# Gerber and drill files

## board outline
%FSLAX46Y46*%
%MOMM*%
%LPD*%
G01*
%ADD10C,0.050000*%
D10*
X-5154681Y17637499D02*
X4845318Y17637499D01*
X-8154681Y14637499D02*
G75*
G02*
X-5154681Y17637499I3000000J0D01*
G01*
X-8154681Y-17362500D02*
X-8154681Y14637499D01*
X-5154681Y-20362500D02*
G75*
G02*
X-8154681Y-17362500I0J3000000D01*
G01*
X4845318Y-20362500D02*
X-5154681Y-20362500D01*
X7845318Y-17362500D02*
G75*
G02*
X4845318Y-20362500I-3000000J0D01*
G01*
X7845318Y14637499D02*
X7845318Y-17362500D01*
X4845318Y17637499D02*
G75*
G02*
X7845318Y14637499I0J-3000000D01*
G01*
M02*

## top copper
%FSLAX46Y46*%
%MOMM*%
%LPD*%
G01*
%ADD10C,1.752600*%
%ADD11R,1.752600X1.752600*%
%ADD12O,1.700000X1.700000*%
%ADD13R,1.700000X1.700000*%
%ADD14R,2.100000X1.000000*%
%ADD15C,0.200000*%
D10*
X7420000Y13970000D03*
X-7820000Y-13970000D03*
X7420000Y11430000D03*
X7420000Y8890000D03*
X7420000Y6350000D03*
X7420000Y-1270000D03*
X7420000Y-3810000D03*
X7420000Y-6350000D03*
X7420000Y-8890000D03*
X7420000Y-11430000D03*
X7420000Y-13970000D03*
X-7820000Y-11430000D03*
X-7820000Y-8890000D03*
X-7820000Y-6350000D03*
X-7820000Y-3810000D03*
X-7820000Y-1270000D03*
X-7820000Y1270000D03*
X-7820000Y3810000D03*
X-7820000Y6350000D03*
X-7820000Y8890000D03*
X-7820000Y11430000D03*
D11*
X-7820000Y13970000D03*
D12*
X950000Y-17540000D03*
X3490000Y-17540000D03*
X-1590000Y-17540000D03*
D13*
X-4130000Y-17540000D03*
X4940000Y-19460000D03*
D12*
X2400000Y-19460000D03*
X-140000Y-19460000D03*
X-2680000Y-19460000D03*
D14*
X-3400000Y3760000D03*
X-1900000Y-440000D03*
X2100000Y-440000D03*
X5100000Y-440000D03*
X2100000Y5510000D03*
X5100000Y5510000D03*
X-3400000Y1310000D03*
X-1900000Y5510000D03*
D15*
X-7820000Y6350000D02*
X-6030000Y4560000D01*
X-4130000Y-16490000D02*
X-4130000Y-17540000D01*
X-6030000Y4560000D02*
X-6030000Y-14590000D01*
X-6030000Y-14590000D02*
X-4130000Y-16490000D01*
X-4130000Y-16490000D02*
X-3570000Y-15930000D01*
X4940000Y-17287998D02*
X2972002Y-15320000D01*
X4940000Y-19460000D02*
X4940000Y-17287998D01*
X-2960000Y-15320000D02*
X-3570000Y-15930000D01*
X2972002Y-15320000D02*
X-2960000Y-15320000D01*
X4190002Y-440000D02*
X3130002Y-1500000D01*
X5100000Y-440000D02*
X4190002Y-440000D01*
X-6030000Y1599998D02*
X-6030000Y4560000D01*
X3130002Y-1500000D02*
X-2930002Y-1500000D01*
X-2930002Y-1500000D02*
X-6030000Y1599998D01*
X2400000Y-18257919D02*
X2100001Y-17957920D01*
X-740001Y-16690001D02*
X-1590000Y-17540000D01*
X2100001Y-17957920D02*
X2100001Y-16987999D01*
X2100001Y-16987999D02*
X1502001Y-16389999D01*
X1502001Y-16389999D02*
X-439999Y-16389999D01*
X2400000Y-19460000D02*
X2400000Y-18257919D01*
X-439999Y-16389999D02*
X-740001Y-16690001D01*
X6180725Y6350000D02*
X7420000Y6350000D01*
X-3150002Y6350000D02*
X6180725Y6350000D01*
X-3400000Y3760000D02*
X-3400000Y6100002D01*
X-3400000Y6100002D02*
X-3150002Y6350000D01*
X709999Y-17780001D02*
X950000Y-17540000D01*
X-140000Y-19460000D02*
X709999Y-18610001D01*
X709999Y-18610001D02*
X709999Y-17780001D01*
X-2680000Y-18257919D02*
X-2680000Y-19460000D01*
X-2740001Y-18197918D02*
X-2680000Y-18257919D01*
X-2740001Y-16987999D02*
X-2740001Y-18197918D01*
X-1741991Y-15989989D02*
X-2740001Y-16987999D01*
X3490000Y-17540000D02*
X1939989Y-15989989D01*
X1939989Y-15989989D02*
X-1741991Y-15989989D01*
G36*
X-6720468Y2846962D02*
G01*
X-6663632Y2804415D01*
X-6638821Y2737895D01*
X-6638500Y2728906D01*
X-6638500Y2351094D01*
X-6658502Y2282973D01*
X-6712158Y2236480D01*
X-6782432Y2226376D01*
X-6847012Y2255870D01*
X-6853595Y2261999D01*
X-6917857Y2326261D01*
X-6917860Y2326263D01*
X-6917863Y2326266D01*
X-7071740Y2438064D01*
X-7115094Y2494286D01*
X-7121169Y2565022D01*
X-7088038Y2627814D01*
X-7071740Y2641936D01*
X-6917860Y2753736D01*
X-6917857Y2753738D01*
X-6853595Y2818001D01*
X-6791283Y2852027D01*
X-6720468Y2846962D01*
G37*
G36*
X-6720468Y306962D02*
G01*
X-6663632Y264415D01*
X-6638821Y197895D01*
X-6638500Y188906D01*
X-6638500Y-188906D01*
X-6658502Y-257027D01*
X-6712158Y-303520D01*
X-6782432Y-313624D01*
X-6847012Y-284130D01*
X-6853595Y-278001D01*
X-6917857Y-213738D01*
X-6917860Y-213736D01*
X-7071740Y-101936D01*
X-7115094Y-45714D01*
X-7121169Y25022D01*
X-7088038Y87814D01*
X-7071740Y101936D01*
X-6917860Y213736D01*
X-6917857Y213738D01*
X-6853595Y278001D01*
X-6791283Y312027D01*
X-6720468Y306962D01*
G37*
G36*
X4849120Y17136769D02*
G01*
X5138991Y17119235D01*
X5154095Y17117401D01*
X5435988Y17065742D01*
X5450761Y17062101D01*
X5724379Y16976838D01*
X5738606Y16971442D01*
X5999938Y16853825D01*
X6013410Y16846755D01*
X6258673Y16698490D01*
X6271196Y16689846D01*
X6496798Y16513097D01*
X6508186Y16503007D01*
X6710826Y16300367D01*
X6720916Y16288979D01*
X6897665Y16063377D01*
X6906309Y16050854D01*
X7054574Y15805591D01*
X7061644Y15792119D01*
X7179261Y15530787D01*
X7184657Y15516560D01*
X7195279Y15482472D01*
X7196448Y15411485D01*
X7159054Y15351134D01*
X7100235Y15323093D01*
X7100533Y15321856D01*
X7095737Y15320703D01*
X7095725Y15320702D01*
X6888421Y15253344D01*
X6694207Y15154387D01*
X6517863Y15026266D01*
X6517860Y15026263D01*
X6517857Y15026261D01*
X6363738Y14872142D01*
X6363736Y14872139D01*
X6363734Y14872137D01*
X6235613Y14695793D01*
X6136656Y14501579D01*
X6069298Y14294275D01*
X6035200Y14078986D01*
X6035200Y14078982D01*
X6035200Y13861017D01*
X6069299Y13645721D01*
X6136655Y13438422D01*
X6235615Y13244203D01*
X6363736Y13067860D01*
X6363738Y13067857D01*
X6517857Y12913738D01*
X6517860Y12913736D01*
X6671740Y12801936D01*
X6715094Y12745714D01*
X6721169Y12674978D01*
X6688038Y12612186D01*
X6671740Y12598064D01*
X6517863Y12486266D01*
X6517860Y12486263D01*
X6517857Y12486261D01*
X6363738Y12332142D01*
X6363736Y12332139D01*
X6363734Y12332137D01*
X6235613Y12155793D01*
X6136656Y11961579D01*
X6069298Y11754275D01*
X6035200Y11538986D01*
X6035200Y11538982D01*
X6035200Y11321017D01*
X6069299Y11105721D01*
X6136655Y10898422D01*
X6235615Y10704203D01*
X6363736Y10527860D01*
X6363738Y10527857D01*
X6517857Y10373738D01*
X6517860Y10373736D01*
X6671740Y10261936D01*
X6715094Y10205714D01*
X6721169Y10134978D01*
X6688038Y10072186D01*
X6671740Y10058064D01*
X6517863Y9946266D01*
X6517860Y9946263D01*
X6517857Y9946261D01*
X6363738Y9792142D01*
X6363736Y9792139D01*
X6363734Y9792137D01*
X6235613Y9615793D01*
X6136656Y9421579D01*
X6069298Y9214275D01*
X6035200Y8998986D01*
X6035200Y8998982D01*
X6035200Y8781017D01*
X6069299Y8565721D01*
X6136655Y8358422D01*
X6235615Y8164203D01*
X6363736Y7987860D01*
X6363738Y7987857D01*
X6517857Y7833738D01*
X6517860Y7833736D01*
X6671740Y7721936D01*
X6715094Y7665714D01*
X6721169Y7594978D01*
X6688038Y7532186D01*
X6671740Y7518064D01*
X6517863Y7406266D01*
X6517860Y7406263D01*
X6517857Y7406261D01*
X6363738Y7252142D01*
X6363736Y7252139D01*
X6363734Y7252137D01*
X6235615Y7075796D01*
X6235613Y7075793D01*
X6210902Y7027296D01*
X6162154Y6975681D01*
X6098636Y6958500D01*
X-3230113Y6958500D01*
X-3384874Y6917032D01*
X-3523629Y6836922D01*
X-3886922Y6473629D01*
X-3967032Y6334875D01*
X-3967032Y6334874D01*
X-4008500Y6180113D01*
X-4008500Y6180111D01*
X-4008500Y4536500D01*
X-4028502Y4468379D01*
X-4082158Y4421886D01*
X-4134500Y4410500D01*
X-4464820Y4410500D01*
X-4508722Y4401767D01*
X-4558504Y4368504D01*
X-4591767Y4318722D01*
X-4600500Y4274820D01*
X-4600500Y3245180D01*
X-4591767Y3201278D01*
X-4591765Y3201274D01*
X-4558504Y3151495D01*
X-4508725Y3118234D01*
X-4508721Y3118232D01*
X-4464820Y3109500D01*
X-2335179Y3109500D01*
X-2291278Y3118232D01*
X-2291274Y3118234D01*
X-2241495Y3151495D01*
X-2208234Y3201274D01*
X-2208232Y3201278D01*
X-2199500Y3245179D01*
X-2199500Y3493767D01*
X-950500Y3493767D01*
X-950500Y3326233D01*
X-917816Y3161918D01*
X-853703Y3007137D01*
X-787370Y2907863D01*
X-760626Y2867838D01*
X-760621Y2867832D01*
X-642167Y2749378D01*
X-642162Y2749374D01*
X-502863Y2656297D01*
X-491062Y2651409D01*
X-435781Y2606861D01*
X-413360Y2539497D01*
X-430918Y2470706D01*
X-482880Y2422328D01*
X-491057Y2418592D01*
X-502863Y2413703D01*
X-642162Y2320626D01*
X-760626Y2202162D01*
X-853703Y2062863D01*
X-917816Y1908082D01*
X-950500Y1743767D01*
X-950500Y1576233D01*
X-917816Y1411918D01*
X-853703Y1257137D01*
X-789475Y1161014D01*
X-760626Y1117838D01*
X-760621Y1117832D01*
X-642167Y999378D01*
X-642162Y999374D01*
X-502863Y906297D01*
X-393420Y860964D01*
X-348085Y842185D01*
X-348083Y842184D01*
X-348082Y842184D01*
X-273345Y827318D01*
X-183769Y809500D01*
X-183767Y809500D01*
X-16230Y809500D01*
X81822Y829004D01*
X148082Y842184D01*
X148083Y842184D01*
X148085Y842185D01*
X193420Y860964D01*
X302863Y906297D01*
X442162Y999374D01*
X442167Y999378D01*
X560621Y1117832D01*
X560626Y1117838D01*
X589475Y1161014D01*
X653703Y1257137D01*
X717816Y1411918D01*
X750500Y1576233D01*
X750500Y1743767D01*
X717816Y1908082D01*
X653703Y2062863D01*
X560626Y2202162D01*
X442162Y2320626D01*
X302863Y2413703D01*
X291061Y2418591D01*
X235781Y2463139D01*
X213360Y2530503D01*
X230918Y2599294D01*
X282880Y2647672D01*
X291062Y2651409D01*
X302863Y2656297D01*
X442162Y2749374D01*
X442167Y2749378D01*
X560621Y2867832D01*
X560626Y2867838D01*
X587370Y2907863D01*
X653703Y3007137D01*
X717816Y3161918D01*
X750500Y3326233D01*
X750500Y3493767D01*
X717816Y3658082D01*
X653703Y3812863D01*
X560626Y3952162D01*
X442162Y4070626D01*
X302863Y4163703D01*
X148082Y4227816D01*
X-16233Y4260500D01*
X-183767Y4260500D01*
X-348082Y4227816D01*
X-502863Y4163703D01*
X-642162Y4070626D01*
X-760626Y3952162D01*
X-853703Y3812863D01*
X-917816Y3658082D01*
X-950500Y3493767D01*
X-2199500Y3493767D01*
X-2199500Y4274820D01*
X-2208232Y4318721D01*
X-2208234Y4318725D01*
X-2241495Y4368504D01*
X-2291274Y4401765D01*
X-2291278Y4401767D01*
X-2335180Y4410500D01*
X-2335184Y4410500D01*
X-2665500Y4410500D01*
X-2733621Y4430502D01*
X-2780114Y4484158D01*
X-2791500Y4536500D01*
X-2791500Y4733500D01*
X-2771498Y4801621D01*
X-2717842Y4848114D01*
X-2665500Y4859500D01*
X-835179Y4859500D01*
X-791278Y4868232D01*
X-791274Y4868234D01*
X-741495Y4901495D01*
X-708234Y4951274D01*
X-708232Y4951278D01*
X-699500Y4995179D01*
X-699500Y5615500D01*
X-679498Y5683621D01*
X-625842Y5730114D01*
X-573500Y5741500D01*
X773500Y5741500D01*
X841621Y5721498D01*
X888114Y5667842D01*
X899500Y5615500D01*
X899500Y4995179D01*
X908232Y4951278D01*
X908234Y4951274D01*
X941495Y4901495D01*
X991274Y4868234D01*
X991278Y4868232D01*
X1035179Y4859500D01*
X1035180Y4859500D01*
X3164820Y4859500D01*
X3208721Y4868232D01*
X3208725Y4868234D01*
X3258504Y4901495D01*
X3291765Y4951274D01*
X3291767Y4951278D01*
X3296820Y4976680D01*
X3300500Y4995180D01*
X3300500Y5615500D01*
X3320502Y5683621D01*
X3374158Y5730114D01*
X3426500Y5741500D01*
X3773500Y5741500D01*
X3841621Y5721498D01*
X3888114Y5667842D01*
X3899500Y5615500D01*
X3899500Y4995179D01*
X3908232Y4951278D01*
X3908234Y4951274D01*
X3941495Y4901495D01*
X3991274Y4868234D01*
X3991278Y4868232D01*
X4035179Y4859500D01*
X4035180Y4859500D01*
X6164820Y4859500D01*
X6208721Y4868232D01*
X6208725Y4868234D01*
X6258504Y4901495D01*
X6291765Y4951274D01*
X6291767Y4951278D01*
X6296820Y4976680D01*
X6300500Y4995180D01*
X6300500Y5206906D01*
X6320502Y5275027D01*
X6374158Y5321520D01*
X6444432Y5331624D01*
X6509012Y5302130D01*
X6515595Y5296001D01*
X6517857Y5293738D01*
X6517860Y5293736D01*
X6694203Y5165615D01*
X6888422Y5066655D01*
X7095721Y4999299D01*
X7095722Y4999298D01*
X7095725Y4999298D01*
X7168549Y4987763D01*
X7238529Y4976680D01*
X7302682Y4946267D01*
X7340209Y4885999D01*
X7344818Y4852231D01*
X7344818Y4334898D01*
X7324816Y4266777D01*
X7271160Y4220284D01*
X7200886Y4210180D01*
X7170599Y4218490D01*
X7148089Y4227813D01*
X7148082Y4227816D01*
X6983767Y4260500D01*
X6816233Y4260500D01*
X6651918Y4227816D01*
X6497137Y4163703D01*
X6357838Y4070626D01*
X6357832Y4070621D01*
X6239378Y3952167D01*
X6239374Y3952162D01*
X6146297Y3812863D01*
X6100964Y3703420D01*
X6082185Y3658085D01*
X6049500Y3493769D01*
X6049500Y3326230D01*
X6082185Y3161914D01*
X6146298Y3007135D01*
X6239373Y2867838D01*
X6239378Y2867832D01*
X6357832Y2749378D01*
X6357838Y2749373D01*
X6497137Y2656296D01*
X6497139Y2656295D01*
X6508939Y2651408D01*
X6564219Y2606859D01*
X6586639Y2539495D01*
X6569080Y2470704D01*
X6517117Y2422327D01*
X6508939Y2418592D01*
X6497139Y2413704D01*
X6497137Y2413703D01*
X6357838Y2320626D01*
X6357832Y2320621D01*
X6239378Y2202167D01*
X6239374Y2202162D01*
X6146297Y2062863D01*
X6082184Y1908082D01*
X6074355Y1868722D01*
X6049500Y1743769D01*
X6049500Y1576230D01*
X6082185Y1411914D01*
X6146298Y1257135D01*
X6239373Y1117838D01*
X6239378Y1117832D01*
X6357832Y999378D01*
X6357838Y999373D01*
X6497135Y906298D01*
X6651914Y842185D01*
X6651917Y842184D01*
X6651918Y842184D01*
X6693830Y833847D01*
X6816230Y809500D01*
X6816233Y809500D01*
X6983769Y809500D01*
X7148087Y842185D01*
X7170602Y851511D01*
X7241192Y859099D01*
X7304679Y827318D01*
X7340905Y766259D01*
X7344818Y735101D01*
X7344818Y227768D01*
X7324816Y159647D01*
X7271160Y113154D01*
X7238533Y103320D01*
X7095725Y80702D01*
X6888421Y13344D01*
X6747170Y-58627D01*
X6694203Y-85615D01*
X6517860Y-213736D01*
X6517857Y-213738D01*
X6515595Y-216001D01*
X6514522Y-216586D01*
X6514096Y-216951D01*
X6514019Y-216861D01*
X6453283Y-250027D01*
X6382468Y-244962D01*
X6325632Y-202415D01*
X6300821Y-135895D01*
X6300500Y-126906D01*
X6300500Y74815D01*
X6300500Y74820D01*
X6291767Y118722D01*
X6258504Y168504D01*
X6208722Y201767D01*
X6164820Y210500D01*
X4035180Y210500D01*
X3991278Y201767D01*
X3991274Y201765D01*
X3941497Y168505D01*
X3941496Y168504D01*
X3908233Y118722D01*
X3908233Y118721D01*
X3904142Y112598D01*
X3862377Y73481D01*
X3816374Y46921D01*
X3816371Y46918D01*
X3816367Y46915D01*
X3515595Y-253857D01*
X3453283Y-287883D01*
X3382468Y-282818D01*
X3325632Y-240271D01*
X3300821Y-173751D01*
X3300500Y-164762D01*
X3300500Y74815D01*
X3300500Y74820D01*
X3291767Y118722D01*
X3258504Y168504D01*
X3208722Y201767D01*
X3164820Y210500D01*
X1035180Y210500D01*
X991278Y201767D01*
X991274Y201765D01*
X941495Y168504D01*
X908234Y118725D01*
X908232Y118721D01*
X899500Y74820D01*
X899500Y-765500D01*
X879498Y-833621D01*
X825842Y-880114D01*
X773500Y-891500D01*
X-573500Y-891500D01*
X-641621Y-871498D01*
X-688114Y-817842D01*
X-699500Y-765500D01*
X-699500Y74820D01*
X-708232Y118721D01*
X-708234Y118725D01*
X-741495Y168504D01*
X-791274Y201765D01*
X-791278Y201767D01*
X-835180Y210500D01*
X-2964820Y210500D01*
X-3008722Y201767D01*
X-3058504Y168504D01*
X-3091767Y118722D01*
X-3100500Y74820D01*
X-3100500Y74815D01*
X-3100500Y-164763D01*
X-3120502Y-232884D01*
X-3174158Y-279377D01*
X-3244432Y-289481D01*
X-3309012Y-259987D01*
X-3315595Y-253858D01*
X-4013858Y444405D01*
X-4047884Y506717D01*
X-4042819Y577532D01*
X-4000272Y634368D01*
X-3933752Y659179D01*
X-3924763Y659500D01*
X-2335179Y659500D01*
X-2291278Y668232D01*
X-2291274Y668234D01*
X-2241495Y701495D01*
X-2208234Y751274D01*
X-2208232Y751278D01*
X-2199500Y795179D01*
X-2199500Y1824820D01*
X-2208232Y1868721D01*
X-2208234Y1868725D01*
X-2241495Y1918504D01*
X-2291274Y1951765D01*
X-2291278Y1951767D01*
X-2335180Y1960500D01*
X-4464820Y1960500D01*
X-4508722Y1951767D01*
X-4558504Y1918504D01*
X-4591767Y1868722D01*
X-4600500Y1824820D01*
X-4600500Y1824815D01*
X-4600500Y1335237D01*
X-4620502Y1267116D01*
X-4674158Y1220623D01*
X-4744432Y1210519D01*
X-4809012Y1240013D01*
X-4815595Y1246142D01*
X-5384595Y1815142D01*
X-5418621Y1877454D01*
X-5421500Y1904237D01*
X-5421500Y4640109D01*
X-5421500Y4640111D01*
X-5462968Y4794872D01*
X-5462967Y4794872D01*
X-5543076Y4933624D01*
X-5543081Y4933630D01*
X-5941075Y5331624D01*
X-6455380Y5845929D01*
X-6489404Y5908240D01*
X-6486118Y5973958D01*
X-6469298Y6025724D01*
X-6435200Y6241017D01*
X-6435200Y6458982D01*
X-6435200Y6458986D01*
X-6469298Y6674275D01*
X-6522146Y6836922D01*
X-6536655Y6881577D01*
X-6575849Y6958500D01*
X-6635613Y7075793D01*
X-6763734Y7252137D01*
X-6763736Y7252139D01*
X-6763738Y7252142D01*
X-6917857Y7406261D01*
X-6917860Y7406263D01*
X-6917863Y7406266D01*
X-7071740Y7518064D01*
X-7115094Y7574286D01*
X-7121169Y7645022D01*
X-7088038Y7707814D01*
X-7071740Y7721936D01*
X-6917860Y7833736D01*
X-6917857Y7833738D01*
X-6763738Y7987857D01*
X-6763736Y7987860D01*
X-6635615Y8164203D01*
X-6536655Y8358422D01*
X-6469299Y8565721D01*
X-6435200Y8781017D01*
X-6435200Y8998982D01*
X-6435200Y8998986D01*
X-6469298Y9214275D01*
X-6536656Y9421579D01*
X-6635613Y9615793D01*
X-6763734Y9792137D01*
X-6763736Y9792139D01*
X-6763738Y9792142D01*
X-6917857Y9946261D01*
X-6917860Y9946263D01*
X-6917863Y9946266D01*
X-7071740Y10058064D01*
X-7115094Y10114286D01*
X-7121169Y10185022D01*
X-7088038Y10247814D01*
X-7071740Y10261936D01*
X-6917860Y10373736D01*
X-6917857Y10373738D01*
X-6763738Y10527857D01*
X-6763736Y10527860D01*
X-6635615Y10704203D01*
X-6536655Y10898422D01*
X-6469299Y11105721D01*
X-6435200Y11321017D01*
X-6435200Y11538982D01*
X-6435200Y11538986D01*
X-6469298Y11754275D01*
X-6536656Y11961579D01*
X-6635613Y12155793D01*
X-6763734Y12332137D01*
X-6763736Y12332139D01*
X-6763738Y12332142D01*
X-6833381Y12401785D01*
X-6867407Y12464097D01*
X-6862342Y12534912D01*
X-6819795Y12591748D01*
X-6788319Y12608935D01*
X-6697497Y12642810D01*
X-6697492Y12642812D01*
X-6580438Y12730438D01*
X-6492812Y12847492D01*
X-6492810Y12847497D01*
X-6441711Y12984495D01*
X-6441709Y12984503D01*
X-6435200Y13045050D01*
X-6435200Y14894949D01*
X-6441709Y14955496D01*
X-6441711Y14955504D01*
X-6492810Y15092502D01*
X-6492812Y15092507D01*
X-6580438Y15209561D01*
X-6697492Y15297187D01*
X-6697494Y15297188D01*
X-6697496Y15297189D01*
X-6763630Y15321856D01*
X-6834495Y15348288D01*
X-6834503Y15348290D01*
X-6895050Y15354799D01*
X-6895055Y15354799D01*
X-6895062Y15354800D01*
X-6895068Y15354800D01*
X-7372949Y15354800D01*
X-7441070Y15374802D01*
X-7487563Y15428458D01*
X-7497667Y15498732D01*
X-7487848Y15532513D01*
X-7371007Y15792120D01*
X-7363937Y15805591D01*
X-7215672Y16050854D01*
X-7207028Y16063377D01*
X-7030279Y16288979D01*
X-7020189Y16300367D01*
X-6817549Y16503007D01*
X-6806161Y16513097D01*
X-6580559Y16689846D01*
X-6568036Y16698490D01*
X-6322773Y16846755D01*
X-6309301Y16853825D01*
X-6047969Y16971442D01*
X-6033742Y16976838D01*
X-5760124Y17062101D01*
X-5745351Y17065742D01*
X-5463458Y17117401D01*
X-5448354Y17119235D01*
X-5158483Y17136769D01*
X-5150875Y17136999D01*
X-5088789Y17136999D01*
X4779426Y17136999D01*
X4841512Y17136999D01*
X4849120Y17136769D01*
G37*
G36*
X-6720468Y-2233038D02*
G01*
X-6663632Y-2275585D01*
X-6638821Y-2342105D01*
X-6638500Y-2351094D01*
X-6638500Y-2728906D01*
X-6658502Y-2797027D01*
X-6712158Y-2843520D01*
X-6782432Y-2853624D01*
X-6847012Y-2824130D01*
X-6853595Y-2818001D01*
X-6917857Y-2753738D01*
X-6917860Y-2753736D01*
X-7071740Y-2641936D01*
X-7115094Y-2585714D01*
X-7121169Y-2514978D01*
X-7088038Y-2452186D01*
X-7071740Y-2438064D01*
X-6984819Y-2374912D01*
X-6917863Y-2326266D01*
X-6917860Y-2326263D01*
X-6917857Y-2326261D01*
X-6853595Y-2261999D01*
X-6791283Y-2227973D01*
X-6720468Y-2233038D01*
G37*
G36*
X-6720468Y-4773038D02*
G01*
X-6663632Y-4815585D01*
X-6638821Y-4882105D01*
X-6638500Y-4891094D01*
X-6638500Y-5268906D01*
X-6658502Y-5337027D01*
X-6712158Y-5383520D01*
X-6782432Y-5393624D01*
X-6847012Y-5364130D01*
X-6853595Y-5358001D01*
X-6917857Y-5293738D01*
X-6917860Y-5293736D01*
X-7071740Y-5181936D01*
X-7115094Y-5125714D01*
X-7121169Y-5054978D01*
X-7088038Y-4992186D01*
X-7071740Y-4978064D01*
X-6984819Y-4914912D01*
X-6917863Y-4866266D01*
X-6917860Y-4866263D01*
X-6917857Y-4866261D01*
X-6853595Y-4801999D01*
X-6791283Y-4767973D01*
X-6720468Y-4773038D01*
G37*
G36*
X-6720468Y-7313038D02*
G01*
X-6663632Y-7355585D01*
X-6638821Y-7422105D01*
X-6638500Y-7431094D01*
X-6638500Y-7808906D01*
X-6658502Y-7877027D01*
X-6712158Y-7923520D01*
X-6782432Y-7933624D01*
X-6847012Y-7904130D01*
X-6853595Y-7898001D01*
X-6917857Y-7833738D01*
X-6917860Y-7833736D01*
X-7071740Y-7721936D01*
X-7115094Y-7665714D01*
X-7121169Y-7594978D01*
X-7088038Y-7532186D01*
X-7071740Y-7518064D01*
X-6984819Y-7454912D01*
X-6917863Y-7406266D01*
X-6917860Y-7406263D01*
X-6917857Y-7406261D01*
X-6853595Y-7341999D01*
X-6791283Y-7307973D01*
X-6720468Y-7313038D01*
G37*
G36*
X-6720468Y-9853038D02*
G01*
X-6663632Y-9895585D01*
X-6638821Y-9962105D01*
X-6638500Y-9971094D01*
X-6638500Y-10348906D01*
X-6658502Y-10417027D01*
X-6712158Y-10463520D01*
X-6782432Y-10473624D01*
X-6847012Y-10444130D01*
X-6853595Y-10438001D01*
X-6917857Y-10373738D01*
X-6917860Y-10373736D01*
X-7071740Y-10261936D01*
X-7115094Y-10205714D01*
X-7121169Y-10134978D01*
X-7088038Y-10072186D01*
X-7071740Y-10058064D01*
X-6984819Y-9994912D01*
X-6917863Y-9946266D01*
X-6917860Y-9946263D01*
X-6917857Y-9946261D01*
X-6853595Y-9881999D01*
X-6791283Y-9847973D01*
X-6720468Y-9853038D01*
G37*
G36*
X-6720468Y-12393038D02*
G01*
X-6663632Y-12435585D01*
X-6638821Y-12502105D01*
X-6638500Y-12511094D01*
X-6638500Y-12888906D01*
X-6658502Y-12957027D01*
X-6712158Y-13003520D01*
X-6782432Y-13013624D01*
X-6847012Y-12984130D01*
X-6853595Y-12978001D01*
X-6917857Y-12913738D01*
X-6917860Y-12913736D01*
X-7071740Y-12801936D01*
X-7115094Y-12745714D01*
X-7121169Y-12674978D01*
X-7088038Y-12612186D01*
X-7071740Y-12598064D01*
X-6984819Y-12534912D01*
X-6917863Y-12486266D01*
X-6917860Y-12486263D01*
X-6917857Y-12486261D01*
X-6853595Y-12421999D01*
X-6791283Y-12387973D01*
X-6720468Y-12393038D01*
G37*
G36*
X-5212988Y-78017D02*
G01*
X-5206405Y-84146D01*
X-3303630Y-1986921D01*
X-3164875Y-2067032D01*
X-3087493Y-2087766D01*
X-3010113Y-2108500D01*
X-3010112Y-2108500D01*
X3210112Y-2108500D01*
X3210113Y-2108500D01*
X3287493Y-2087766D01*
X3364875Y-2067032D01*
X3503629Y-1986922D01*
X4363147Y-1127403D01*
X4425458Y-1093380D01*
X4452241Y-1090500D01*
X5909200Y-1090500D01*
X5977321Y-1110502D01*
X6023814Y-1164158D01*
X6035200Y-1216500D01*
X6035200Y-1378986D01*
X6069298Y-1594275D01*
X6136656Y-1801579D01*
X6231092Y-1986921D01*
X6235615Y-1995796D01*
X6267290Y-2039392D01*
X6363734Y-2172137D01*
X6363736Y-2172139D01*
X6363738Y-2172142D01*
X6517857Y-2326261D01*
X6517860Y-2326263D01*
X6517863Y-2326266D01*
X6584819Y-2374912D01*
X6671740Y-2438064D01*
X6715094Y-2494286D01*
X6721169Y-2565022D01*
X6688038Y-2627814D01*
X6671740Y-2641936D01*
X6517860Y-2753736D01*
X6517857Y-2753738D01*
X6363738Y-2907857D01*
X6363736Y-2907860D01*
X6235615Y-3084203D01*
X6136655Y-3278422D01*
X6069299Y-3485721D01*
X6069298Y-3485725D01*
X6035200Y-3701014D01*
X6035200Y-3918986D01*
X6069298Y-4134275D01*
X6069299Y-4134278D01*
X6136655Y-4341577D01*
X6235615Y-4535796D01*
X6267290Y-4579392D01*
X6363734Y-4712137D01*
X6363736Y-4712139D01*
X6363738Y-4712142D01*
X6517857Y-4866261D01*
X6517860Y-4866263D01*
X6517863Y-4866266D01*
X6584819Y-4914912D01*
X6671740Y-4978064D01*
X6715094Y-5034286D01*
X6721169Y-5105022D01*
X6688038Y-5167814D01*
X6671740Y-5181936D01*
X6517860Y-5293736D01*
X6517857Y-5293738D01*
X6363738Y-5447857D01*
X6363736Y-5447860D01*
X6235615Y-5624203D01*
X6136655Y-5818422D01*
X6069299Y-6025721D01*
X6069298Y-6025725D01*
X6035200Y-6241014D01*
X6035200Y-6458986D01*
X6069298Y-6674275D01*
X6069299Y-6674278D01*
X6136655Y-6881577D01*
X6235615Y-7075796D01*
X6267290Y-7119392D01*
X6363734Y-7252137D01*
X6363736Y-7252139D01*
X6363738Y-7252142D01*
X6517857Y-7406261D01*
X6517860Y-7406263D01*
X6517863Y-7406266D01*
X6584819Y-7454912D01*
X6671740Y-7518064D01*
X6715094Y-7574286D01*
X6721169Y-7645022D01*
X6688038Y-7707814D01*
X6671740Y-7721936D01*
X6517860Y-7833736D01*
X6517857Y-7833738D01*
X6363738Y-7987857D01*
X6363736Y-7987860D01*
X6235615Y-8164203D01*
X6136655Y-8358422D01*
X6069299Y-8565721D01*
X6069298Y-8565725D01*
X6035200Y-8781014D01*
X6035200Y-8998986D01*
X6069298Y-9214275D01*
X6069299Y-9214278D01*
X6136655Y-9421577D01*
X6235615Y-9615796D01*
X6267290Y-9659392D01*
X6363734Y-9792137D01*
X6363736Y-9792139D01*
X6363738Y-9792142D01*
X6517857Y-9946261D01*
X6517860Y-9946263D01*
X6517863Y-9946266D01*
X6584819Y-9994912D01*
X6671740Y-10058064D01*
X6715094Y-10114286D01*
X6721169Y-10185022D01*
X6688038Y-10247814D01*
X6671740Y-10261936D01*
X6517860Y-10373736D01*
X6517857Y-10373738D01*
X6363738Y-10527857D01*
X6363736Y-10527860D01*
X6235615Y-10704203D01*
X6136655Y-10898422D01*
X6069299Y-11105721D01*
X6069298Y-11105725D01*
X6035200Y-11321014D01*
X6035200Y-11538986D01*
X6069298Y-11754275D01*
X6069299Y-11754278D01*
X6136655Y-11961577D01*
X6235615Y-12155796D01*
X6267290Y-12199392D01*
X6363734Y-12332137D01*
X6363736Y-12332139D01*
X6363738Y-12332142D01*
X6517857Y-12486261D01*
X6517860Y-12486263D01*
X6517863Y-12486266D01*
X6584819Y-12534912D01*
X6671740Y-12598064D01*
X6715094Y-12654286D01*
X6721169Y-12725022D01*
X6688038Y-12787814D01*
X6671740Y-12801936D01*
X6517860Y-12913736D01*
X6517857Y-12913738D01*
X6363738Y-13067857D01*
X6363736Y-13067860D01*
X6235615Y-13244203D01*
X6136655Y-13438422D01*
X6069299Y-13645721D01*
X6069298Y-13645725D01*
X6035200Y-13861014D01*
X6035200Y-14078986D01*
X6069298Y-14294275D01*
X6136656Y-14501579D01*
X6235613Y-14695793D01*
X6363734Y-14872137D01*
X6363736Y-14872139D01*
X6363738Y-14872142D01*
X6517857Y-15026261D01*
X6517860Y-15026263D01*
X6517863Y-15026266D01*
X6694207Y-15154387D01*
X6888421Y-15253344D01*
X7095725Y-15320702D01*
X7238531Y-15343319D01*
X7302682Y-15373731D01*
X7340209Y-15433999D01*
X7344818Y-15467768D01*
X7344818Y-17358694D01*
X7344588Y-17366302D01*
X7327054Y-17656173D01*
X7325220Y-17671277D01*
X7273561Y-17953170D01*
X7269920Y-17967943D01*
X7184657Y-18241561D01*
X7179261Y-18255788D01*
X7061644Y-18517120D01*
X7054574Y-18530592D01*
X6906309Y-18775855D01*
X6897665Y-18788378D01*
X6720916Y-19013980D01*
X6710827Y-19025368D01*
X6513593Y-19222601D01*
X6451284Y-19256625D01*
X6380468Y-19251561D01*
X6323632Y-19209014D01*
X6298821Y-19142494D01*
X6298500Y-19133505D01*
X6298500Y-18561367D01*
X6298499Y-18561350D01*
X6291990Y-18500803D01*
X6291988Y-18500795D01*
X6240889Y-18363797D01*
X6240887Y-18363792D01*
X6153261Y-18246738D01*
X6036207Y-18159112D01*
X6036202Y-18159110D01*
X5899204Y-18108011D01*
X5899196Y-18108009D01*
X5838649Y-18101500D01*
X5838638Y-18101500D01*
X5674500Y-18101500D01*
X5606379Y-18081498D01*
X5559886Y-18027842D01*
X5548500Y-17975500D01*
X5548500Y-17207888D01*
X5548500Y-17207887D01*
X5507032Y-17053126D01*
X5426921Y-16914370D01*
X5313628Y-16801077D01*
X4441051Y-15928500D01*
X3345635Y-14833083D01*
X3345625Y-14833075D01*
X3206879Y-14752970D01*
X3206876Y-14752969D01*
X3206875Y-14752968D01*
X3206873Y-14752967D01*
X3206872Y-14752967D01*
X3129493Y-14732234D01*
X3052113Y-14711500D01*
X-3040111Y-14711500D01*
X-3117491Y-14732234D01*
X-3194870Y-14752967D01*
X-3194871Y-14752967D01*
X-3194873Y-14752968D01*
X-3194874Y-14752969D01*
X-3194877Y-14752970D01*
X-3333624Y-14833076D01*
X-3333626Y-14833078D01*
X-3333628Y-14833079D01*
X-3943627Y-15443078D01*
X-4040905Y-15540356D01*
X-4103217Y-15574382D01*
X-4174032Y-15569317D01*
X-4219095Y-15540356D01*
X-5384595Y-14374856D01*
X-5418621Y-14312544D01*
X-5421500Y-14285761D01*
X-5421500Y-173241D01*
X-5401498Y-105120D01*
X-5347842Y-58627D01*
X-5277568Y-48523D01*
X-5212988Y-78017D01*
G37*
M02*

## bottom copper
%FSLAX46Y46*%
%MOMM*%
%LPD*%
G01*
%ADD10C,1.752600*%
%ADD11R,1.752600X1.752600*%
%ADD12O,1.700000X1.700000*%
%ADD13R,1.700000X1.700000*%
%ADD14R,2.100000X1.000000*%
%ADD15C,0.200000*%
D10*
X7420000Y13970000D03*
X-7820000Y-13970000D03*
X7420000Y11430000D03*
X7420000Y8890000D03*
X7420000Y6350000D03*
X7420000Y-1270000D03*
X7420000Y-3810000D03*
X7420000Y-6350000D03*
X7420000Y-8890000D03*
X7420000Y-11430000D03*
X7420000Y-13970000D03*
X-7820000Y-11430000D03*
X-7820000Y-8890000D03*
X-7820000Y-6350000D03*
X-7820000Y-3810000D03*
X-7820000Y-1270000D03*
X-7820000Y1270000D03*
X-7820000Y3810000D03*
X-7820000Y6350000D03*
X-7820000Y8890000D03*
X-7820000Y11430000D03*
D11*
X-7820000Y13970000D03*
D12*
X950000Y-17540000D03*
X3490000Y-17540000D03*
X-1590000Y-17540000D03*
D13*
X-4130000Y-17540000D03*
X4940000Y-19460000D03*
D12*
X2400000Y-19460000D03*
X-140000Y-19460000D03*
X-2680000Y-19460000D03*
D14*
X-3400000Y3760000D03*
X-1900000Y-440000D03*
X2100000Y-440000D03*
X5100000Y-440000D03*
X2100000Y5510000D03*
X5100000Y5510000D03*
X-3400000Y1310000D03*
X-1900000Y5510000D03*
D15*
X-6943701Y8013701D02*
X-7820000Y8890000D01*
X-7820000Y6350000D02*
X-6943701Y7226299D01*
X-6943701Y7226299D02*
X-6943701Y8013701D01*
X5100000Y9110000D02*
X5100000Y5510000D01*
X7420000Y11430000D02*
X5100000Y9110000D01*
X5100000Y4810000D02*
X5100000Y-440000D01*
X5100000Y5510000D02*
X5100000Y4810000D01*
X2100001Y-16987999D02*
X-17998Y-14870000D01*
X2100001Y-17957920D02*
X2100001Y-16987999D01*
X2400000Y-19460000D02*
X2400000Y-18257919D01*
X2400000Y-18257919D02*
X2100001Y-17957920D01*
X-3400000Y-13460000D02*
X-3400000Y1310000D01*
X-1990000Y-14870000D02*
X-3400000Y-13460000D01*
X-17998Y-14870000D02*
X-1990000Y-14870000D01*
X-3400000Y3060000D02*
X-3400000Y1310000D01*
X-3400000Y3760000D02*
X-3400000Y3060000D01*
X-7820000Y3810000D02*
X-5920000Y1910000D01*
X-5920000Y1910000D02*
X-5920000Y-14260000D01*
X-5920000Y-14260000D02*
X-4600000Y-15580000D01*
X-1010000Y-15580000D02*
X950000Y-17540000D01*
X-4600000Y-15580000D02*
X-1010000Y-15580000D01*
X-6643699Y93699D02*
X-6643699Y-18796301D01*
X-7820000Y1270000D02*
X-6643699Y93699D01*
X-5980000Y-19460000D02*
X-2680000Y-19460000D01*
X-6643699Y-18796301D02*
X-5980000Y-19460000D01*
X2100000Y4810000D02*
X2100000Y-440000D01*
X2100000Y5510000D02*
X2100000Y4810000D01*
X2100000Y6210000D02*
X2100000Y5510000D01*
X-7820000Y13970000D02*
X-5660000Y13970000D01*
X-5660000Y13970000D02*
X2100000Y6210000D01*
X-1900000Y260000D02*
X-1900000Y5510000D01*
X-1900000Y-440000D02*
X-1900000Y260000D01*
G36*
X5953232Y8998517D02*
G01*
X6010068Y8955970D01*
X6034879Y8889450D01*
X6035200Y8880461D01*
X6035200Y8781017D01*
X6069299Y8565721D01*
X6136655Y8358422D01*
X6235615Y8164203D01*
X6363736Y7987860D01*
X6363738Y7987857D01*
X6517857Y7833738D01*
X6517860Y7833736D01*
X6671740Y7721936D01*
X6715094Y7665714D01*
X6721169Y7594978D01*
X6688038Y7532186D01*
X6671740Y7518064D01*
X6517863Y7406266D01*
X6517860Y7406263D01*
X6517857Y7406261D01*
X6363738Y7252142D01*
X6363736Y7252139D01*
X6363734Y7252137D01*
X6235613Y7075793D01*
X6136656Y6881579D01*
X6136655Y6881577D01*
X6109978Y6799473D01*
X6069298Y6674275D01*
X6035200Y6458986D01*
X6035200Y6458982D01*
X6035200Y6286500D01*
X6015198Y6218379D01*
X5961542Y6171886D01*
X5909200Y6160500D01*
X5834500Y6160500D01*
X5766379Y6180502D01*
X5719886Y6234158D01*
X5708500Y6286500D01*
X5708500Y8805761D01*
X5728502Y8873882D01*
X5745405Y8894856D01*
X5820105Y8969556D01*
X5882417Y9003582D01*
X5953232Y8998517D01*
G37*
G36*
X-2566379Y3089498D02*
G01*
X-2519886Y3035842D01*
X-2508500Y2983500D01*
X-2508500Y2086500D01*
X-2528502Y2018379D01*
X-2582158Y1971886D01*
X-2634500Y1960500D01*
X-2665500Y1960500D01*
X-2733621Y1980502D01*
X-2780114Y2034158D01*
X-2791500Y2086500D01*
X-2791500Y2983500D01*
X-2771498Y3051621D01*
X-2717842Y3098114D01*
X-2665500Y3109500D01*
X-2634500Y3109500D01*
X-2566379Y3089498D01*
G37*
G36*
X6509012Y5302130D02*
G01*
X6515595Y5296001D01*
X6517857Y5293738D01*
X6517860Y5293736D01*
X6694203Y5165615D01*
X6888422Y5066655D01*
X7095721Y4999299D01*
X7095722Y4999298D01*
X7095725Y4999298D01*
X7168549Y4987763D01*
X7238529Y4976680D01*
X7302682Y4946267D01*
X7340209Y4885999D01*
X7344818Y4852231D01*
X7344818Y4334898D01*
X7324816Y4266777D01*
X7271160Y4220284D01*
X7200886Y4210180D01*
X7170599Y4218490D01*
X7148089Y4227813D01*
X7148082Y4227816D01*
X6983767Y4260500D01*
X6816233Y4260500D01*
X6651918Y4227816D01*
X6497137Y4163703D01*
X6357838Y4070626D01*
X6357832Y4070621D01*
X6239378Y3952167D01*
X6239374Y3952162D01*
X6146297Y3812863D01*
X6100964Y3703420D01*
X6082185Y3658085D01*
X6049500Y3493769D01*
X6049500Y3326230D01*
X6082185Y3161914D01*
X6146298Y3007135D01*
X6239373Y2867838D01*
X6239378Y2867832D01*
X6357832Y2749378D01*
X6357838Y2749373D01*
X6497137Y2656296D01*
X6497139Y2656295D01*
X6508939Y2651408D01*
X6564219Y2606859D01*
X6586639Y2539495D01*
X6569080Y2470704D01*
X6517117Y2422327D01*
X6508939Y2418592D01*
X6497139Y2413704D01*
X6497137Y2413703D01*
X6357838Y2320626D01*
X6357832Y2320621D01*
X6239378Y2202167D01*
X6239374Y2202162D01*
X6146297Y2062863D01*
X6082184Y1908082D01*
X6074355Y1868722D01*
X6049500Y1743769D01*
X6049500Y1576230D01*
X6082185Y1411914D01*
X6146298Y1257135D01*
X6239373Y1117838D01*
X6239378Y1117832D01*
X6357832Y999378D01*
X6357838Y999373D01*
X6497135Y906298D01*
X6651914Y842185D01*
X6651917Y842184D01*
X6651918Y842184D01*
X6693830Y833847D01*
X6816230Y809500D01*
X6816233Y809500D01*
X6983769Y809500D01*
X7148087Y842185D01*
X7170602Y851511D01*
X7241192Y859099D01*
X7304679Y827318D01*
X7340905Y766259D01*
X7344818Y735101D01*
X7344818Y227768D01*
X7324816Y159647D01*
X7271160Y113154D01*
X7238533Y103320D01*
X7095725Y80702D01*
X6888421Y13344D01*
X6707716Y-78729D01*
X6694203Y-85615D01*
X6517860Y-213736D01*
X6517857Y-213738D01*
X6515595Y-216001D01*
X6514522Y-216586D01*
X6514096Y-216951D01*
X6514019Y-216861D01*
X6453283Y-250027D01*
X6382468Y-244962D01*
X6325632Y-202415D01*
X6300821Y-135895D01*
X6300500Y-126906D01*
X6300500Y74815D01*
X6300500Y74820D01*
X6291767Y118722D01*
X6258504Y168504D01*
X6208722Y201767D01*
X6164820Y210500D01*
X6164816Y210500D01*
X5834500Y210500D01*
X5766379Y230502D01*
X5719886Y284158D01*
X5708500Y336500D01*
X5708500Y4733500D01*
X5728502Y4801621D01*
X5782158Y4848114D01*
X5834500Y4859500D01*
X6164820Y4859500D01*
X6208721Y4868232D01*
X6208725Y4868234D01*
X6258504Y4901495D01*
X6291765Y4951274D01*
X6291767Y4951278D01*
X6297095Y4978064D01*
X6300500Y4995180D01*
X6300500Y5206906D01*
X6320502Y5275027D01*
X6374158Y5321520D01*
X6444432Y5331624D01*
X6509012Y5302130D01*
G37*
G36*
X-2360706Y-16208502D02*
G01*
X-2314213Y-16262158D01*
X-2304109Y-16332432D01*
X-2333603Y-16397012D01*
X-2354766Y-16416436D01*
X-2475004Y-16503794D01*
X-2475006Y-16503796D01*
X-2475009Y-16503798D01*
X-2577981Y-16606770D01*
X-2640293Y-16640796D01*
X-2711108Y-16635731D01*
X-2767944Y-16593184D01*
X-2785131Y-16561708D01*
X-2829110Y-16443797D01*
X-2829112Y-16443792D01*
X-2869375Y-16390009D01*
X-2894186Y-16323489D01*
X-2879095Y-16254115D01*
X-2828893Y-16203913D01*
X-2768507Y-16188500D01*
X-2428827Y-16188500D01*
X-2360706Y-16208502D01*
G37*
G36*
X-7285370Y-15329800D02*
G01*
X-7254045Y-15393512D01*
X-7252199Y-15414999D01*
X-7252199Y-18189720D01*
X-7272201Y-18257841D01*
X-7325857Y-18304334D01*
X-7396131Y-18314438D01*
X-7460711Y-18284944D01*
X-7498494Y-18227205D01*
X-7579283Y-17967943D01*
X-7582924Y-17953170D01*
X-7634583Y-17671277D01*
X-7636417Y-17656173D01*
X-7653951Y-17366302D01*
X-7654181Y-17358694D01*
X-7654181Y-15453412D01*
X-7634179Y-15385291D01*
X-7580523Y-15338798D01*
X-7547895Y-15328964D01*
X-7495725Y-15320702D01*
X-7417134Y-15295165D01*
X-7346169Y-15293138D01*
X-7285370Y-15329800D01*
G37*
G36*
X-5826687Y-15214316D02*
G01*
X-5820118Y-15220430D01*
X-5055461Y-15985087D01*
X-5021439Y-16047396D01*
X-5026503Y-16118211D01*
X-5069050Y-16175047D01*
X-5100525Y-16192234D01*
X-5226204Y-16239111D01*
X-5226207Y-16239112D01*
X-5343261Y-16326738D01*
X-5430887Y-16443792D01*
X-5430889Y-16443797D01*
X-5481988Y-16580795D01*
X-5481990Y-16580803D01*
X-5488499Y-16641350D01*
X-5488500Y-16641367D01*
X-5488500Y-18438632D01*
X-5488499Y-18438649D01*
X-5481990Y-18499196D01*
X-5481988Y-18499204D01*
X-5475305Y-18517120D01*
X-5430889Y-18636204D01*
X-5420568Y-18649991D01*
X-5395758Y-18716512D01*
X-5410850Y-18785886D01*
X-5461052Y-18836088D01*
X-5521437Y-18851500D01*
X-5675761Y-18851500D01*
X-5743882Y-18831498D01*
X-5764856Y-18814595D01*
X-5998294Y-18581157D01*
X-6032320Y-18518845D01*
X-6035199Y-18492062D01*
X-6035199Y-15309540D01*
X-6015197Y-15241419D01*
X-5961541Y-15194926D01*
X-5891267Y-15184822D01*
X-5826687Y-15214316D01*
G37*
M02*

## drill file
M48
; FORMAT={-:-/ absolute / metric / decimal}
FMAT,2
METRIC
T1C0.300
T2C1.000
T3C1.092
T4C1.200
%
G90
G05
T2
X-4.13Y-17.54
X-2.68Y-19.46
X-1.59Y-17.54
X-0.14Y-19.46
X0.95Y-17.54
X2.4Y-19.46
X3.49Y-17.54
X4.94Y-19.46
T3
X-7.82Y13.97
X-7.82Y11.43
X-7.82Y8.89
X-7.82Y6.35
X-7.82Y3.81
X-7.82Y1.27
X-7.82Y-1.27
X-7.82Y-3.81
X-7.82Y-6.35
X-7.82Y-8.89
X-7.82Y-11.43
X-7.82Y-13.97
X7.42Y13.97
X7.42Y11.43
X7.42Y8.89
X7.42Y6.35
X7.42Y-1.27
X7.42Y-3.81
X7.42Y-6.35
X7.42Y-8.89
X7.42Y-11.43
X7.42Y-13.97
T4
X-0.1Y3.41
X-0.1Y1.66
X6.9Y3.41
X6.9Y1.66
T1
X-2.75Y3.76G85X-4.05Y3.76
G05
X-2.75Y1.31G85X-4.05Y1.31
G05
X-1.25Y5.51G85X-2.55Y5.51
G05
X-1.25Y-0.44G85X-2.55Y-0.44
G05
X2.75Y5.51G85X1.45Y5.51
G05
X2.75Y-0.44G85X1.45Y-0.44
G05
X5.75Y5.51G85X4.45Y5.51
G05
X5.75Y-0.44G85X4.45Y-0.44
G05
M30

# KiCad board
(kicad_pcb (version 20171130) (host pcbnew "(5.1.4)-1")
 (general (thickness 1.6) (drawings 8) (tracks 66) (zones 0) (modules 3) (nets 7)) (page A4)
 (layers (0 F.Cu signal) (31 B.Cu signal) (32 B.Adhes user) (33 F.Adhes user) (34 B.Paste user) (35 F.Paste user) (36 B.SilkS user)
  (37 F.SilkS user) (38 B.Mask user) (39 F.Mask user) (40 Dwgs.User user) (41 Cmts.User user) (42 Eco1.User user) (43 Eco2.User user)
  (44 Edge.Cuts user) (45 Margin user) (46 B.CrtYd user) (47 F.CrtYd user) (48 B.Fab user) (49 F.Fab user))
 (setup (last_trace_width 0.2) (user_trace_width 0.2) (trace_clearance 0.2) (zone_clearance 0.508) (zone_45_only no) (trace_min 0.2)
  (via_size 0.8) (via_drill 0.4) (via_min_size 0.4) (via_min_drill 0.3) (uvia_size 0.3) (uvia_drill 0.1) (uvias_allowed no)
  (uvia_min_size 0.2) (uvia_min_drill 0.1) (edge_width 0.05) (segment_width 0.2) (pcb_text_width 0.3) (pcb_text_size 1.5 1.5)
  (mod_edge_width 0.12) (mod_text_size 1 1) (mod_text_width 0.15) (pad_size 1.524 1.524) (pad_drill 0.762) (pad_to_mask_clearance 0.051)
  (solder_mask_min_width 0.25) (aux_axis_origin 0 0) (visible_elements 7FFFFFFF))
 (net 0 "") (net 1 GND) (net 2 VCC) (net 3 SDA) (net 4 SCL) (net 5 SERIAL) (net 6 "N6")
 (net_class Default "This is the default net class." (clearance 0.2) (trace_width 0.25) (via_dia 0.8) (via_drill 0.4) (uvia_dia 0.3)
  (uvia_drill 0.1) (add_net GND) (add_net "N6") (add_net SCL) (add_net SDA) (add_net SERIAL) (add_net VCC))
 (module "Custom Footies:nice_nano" (layer F.Cu) (at -0.2 0 270)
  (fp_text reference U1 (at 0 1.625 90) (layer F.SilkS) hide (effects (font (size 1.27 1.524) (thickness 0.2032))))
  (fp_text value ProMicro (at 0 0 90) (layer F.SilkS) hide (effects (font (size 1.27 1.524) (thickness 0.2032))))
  (pad 24 thru_hole circle (at -13.97 -7.62 270) (size 1.7526 1.7526) (drill 1.0922) (layers *.Cu *.SilkS *.Mask))
  (pad 12 thru_hole circle (at 13.97 7.62 270) (size 1.7526 1.7526) (drill 1.0922) (layers *.Cu *.SilkS *.Mask))
  (pad 23 thru_hole circle (at -11.43 -7.62 270) (size 1.7526 1.7526) (drill 1.0922) (layers *.Cu *.SilkS *.Mask) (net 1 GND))
  (pad 22 thru_hole circle (at -8.89 -7.62 270) (size 1.7526 1.7526) (drill 1.0922) (layers *.Cu *.SilkS *.Mask))
  (pad 21 thru_hole circle (at -6.35 -7.62 270) (size 1.7526 1.7526) (drill 1.0922) (layers *.Cu *.SilkS *.Mask) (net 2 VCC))
  (pad 18 thru_hole circle (at 1.27 -7.62 270) (size 1.7526 1.7526) (drill 1.0922) (layers *.Cu *.SilkS *.Mask))
  (pad 17 thru_hole circle (at 3.81 -7.62 270) (size 1.7526 1.7526) (drill 1.0922) (layers *.Cu *.SilkS *.Mask))
  (pad 16 thru_hole circle (at 6.35 -7.62 270) (size 1.7526 1.7526) (drill 1.0922) (layers *.Cu *.SilkS *.Mask))
  (pad 15 thru_hole circle (at 8.89 -7.62 270) (size 1.7526 1.7526) (drill 1.0922) (layers *.Cu *.SilkS *.Mask))
  (pad 14 thru_hole circle (at 11.43 -7.62 270) (size 1.7526 1.7526) (drill 1.0922) (layers *.Cu *.SilkS *.Mask))
  (pad 13 thru_hole circle (at 13.97 -7.62 270) (size 1.7526 1.7526) (drill 1.0922) (layers *.Cu *.SilkS *.Mask))
  (pad 11 thru_hole circle (at 11.43 7.62 270) (size 1.7526 1.7526) (drill 1.0922) (layers *.Cu *.SilkS *.Mask))
  (pad 10 thru_hole circle (at 8.89 7.62 270) (size 1.7526 1.7526) (drill 1.0922) (layers *.Cu *.SilkS *.Mask))
  (pad 9 thru_hole circle (at 6.35 7.62 270) (size 1.7526 1.7526) (drill 1.0922) (layers *.Cu *.SilkS *.Mask))
  (pad 8 thru_hole circle (at 3.81 7.62 270) (size 1.7526 1.7526) (drill 1.0922) (layers *.Cu *.SilkS *.Mask))
  (pad 7 thru_hole circle (at 1.27 7.62 270) (size 1.7526 1.7526) (drill 1.0922) (layers *.Cu *.SilkS *.Mask))
  (pad 6 thru_hole circle (at -1.27 7.62 270) (size 1.7526 1.7526) (drill 1.0922) (layers *.Cu *.SilkS *.Mask) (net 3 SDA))
  (pad 5 thru_hole circle (at -3.81 7.62 270) (size 1.7526 1.7526) (drill 1.0922) (layers *.Cu *.SilkS *.Mask) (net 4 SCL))
  (pad 4 thru_hole circle (at -6.35 7.62 270) (size 1.7526 1.7526) (drill 1.0922) (layers *.Cu *.SilkS *.Mask) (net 1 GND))
  (pad 3 thru_hole circle (at -8.89 7.62 270) (size 1.7526 1.7526) (drill 1.0922) (layers *.Cu *.SilkS *.Mask) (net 1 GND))
  (pad 2 thru_hole circle (at -11.43 7.62 270) (size 1.7526 1.7526) (drill 1.0922) (layers *.Cu *.SilkS *.Mask))
  (pad 1 thru_hole rect (at -13.97 7.62 270) (size 1.7526 1.7526) (drill 1.0922) (layers *.Cu *.SilkS *.Mask) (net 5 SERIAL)))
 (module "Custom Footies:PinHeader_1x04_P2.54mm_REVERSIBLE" (layer F.Cu) (at 4.94 19.46 270)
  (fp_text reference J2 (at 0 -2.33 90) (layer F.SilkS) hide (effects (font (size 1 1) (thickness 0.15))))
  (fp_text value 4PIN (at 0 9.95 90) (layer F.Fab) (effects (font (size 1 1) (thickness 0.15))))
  (pad 3 thru_hole oval (at -1.92 3.99 90) (size 1.7 1.7) (drill 1) (layers *.Cu *.Mask) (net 4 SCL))
  (pad 4 thru_hole oval (at -1.92 1.45 90) (size 1.7 1.7) (drill 1) (layers *.Cu *.Mask) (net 3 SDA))
  (pad 2 thru_hole oval (at -1.92 6.53 90) (size 1.7 1.7) (drill 1) (layers *.Cu *.Mask) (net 2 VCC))
  (pad 1 thru_hole rect (at -1.92 9.07 90) (size 1.7 1.7) (drill 1) (layers *.Cu *.Mask) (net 1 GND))
  (pad 1 thru_hole rect (at 0 0 270) (size 1.7 1.7) (drill 1) (layers *.Cu *.Mask) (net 1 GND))
  (pad 2 thru_hole oval (at 0 2.54 270) (size 1.7 1.7) (drill 1) (layers *.Cu *.Mask) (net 2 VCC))
  (pad 3 thru_hole oval (at 0 5.08 270) (size 1.7 1.7) (drill 1) (layers *.Cu *.Mask) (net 4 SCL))
  (pad 4 thru_hole oval (at 0 7.62 270) (size 1.7 1.7) (drill 1) (layers *.Cu *.Mask) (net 3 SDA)))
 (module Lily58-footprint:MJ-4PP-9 (layer F.Cu) (at 8.4 -1.66 270)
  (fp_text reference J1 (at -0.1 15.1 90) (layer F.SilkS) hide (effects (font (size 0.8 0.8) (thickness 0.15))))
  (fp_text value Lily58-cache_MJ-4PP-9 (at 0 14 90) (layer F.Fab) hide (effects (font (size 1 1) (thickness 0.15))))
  (pad 4 thru_hole rect (at -2.1 11.8 270) (size 1 2.1) (drill oval 0.3 1.6) (layers *.Cu *.Mask F.SilkS) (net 2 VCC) (clearance 0.15))
  (pad 1 thru_hole rect (at 2.1 10.3 270) (size 1 2.1) (drill oval 0.3 1.6) (layers *.Cu *.Mask F.SilkS) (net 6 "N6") (clearance 0.15))
  (pad 2 thru_hole rect (at 2.1 6.3 270) (size 1 2.1) (drill oval 0.3 1.6) (layers *.Cu *.Mask F.SilkS) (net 5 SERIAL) (clearance 0.15))
  (pad 3 thru_hole rect (at 2.1 3.3 270) (size 1 2.1) (drill oval 0.3 1.6) (layers *.Cu *.Mask F.SilkS) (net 1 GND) (clearance 0.15))
  (pad "" np_thru_hole circle (at 0 8.5 270) (size 1.2 1.2) (drill 1.2) (layers *.Cu *.Mask F.SilkS))
  (pad "" np_thru_hole circle (at 0 1.5 270) (size 1.2 1.2) (drill 1.2) (layers *.Cu *.Mask F.SilkS))
  (pad 2 thru_hole rect (at -3.85 6.3 270) (size 1 2.1) (drill oval 0.3 1.6) (layers *.Cu *.Mask F.SilkS) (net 5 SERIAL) (clearance 0.15))
  (pad 3 thru_hole rect (at -3.85 3.3 270) (size 1 2.1) (drill oval 0.3 1.6) (layers *.Cu *.Mask F.SilkS) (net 1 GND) (clearance 0.15))
  (pad 4 thru_hole rect (at 0.35 11.8 270) (size 1 2.1) (drill oval 0.3 1.6) (layers *.Cu *.Mask F.SilkS) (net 2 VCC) (clearance 0.15))
  (pad 1 thru_hole rect (at -3.85 10.3 270) (size 1 2.1) (drill oval 0.3 1.6) (layers *.Cu *.Mask F.SilkS) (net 6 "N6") (clearance 0.15))
  (pad "" np_thru_hole circle (at -1.75 1.5 270) (size 1.2 1.2) (drill 1.2) (layers *.Cu *.Mask F.SilkS))
  (pad "" np_thru_hole circle (at -1.75 8.5 270) (size 1.2 1.2) (drill 1.2) (layers *.Cu *.Mask F.SilkS)))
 (gr_line (start -5.154681 -17.637499) (end 4.845318 -17.637499) (layer Edge.Cuts) (width 0.05))
 (gr_arc (start -5.154681 -14.637499) (end -5.154681 -17.637499) (angle -90) (layer Edge.Cuts) (width 0.05))
 (gr_line (start -8.154681 17.3625) (end -8.154681 -14.637499) (layer Edge.Cuts) (width 0.05))
 (gr_arc (start -5.154681 17.3625) (end -8.154681 17.3625) (angle -90) (layer Edge.Cuts) (width 0.05))
 (gr_line (start 4.845318 20.3625) (end -5.154681 20.3625) (layer Edge.Cuts) (width 0.05))
 (gr_arc (start 4.845318 17.3625) (end 4.845318 20.3625) (angle -90) (layer Edge.Cuts) (width 0.05))
 (gr_line (start 7.845318 -14.637499) (end 7.845318 17.3625) (layer Edge.Cuts) (width 0.05))
 (gr_arc (start 4.845318 -14.637499) (end 7.845318 -14.637499) (angle -90) (layer Edge.Cuts) (width 0.05))
 (segment (start -6.943701 -8.013701) (end -7.82 -8.89) (width 0.2) (layer B.Cu) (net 1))
 (segment (start -7.82 -6.35) (end -6.943701 -7.226299) (width 0.2) (layer B.Cu) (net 1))
 (segment (start -6.943701 -7.226299) (end -6.943701 -8.013701) (width 0.2) (layer B.Cu) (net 1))
 (segment (start -7.82 -6.35) (end -6.03 -4.56) (width 0.2) (layer F.Cu) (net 1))
 (segment (start -4.13 16.49) (end -4.13 17.54) (width 0.2) (layer F.Cu) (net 1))
 (segment (start -6.03 -4.56) (end -6.03 14.59) (width 0.2) (layer F.Cu) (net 1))
 (segment (start -6.03 14.59) (end -4.13 16.49) (width 0.2) (layer F.Cu) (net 1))
 (segment (start -4.13 16.49) (end -3.57 15.93) (width 0.2) (layer F.Cu) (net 1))
 (segment (start 4.94 17.287998) (end 2.972002 15.32) (width 0.2) (layer F.Cu) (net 1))
 (segment (start 4.94 19.46) (end 4.94 17.287998) (width 0.2) (layer F.Cu) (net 1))
 (segment (start -2.96 15.32) (end -3.57 15.93) (width 0.2) (layer F.Cu) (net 1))
 (segment (start 2.972002 15.32) (end -2.96 15.32) (width 0.2) (layer F.Cu) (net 1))
 (segment (start 5.1 -9.11) (end 5.1 -5.51) (width 0.2) (layer B.Cu) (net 1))
 (segment (start 7.42 -11.43) (end 5.1 -9.11) (width 0.2) (layer B.Cu) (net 1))
 (segment (start 5.1 -4.81) (end 5.1 0.44) (width 0.2) (layer B.Cu) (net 1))
 (segment (start 5.1 -5.51) (end 5.1 -4.81) (width 0.2) (layer B.Cu) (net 1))
 (segment (start 4.190002 0.44) (end 3.130002 1.5) (width 0.2) (layer F.Cu) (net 1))
 (segment (start 5.1 0.44) (end 4.190002 0.44) (width 0.2) (layer F.Cu) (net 1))
 (segment (start -6.03 -1.599998) (end -6.03 -4.56) (width 0.2) (layer F.Cu) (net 1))
 (segment (start 3.130002 1.5) (end -2.930002 1.5) (width 0.2) (layer F.Cu) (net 1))
 (segment (start -2.930002 1.5) (end -6.03 -1.599998) (width 0.2) (layer F.Cu) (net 1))
 (segment (start 2.4 18.257919) (end 2.100001 17.95792) (width 0.2) (layer F.Cu) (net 2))
 (segment (start -0.740001 16.690001) (end -1.59 17.54) (width 0.2) (layer F.Cu) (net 2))
 (segment (start 2.100001 17.95792) (end 2.100001 16.987999) (width 0.2) (layer F.Cu) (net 2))
 (segment (start 2.100001 16.987999) (end 1.502001 16.389999) (width 0.2) (layer F.Cu) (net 2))
 (segment (start 1.502001 16.389999) (end -0.439999 16.389999) (width 0.2) (layer F.Cu) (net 2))
 (segment (start 2.4 19.46) (end 2.4 18.257919) (width 0.2) (layer F.Cu) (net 2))
 (segment (start -0.439999 16.389999) (end -0.740001 16.690001) (width 0.2) (layer F.Cu) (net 2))
 (segment (start 2.100001 16.987999) (end -0.017998 14.87) (width 0.2) (layer B.Cu) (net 2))
 (segment (start 2.100001 17.95792) (end 2.100001 16.987999) (width 0.2) (layer B.Cu) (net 2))
 (segment (start 2.4 19.46) (end 2.4 18.257919) (width 0.2) (layer B.Cu) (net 2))
 (segment (start 2.4 18.257919) (end 2.100001 17.95792) (width 0.2) (layer B.Cu) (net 2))
 (segment (start -3.4 13.46) (end -3.4 -1.31) (width 0.2) (layer B.Cu) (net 2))
 (segment (start -1.99 14.87) (end -3.4 13.46) (width 0.2) (layer B.Cu) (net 2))
 (segment (start -0.017998 14.87) (end -1.99 14.87) (width 0.2) (layer B.Cu) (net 2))
 (segment (start -3.4 -3.06) (end -3.4 -1.31) (width 0.2) (layer B.Cu) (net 2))
 (segment (start -3.4 -3.76) (end -3.4 -3.06) (width 0.2) (layer B.Cu) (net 2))
 (segment (start 6.180725 -6.35) (end 7.42 -6.35) (width 0.2) (layer F.Cu) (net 2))
 (segment (start -3.150002 -6.35) (end 6.180725 -6.35) (width 0.2) (layer F.Cu) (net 2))
 (segment (start -3.4 -3.76) (end -3.4 -6.100002) (width 0.2) (layer F.Cu) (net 2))
 (segment (start -3.4 -6.100002) (end -3.150002 -6.35) (width 0.2) (layer F.Cu) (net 2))
 (segment (start -7.82 -3.81) (end -5.92 -1.91) (width 0.2) (layer B.Cu) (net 4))
 (segment (start -5.92 -1.91) (end -5.92 14.26) (width 0.2) (layer B.Cu) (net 4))
 (segment (start -5.92 14.26) (end -4.6 15.58) (width 0.2) (layer B.Cu) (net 4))
 (segment (start -1.01 15.58) (end 0.95 17.54) (width 0.2) (layer B.Cu) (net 4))
 (segment (start -4.6 15.58) (end -1.01 15.58) (width 0.2) (layer B.Cu) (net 4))
 (segment (start 0.709999 17.780001) (end 0.95 17.54) (width 0.2) (layer F.Cu) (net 4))
 (segment (start -0.14 19.46) (end 0.709999 18.610001) (width 0.2) (layer F.Cu) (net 4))
 (segment (start 0.709999 18.610001) (end 0.709999 17.780001) (width 0.2) (layer F.Cu) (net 4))
 (segment (start -6.643699 -0.093699) (end -6.643699 18.796301) (width 0.2) (layer B.Cu) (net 3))
 (segment (start -7.82 -1.27) (end -6.643699 -0.093699) (width 0.2) (layer B.Cu) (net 3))
 (segment (start -5.98 19.46) (end -2.68 19.46) (width 0.2) (layer B.Cu) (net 3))
 (segment (start -6.643699 18.796301) (end -5.98 19.46) (width 0.2) (layer B.Cu) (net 3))
 (segment (start -2.68 18.257919) (end -2.68 19.46) (width 0.2) (layer F.Cu) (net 3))
 (segment (start -2.740001 18.197918) (end -2.68 18.257919) (width 0.2) (layer F.Cu) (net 3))
 (segment (start -2.740001 16.987999) (end -2.740001 18.197918) (width 0.2) (layer F.Cu) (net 3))
 (segment (start -1.741991 15.989989) (end -2.740001 16.987999) (width 0.2) (layer F.Cu) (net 3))
 (segment (start 3.49 17.54) (end 1.939989 15.989989) (width 0.2) (layer F.Cu) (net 3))
 (segment (start 1.939989 15.989989) (end -1.741991 15.989989) (width 0.2) (layer F.Cu) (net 3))
 (segment (start 2.1 -4.81) (end 2.1 0.44) (width 0.2) (layer B.Cu) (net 5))
 (segment (start 2.1 -5.51) (end 2.1 -4.81) (width 0.2) (layer B.Cu) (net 5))
 (segment (start 2.1 -6.21) (end 2.1 -5.51) (width 0.2) (layer B.Cu) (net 5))
 (segment (start -7.82 -13.97) (end -5.66 -13.97) (width 0.2) (layer B.Cu) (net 5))
 (segment (start -5.66 -13.97) (end 2.1 -6.21) (width 0.2) (layer B.Cu) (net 5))
 (segment (start -1.9 -0.26) (end -1.9 -5.51) (width 0.2) (layer B.Cu) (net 6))
 (segment (start -1.9 0.44) (end -1.9 -0.26) (width 0.2) (layer B.Cu) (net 6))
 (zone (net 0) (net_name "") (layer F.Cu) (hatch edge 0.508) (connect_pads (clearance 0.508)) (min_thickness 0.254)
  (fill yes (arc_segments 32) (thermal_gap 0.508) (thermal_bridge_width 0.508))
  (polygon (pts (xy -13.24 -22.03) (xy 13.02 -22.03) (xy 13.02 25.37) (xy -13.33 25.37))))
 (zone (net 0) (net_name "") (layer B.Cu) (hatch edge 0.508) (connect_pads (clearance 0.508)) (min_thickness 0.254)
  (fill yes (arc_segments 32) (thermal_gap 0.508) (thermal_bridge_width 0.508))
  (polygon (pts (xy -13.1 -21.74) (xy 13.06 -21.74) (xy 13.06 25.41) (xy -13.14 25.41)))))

